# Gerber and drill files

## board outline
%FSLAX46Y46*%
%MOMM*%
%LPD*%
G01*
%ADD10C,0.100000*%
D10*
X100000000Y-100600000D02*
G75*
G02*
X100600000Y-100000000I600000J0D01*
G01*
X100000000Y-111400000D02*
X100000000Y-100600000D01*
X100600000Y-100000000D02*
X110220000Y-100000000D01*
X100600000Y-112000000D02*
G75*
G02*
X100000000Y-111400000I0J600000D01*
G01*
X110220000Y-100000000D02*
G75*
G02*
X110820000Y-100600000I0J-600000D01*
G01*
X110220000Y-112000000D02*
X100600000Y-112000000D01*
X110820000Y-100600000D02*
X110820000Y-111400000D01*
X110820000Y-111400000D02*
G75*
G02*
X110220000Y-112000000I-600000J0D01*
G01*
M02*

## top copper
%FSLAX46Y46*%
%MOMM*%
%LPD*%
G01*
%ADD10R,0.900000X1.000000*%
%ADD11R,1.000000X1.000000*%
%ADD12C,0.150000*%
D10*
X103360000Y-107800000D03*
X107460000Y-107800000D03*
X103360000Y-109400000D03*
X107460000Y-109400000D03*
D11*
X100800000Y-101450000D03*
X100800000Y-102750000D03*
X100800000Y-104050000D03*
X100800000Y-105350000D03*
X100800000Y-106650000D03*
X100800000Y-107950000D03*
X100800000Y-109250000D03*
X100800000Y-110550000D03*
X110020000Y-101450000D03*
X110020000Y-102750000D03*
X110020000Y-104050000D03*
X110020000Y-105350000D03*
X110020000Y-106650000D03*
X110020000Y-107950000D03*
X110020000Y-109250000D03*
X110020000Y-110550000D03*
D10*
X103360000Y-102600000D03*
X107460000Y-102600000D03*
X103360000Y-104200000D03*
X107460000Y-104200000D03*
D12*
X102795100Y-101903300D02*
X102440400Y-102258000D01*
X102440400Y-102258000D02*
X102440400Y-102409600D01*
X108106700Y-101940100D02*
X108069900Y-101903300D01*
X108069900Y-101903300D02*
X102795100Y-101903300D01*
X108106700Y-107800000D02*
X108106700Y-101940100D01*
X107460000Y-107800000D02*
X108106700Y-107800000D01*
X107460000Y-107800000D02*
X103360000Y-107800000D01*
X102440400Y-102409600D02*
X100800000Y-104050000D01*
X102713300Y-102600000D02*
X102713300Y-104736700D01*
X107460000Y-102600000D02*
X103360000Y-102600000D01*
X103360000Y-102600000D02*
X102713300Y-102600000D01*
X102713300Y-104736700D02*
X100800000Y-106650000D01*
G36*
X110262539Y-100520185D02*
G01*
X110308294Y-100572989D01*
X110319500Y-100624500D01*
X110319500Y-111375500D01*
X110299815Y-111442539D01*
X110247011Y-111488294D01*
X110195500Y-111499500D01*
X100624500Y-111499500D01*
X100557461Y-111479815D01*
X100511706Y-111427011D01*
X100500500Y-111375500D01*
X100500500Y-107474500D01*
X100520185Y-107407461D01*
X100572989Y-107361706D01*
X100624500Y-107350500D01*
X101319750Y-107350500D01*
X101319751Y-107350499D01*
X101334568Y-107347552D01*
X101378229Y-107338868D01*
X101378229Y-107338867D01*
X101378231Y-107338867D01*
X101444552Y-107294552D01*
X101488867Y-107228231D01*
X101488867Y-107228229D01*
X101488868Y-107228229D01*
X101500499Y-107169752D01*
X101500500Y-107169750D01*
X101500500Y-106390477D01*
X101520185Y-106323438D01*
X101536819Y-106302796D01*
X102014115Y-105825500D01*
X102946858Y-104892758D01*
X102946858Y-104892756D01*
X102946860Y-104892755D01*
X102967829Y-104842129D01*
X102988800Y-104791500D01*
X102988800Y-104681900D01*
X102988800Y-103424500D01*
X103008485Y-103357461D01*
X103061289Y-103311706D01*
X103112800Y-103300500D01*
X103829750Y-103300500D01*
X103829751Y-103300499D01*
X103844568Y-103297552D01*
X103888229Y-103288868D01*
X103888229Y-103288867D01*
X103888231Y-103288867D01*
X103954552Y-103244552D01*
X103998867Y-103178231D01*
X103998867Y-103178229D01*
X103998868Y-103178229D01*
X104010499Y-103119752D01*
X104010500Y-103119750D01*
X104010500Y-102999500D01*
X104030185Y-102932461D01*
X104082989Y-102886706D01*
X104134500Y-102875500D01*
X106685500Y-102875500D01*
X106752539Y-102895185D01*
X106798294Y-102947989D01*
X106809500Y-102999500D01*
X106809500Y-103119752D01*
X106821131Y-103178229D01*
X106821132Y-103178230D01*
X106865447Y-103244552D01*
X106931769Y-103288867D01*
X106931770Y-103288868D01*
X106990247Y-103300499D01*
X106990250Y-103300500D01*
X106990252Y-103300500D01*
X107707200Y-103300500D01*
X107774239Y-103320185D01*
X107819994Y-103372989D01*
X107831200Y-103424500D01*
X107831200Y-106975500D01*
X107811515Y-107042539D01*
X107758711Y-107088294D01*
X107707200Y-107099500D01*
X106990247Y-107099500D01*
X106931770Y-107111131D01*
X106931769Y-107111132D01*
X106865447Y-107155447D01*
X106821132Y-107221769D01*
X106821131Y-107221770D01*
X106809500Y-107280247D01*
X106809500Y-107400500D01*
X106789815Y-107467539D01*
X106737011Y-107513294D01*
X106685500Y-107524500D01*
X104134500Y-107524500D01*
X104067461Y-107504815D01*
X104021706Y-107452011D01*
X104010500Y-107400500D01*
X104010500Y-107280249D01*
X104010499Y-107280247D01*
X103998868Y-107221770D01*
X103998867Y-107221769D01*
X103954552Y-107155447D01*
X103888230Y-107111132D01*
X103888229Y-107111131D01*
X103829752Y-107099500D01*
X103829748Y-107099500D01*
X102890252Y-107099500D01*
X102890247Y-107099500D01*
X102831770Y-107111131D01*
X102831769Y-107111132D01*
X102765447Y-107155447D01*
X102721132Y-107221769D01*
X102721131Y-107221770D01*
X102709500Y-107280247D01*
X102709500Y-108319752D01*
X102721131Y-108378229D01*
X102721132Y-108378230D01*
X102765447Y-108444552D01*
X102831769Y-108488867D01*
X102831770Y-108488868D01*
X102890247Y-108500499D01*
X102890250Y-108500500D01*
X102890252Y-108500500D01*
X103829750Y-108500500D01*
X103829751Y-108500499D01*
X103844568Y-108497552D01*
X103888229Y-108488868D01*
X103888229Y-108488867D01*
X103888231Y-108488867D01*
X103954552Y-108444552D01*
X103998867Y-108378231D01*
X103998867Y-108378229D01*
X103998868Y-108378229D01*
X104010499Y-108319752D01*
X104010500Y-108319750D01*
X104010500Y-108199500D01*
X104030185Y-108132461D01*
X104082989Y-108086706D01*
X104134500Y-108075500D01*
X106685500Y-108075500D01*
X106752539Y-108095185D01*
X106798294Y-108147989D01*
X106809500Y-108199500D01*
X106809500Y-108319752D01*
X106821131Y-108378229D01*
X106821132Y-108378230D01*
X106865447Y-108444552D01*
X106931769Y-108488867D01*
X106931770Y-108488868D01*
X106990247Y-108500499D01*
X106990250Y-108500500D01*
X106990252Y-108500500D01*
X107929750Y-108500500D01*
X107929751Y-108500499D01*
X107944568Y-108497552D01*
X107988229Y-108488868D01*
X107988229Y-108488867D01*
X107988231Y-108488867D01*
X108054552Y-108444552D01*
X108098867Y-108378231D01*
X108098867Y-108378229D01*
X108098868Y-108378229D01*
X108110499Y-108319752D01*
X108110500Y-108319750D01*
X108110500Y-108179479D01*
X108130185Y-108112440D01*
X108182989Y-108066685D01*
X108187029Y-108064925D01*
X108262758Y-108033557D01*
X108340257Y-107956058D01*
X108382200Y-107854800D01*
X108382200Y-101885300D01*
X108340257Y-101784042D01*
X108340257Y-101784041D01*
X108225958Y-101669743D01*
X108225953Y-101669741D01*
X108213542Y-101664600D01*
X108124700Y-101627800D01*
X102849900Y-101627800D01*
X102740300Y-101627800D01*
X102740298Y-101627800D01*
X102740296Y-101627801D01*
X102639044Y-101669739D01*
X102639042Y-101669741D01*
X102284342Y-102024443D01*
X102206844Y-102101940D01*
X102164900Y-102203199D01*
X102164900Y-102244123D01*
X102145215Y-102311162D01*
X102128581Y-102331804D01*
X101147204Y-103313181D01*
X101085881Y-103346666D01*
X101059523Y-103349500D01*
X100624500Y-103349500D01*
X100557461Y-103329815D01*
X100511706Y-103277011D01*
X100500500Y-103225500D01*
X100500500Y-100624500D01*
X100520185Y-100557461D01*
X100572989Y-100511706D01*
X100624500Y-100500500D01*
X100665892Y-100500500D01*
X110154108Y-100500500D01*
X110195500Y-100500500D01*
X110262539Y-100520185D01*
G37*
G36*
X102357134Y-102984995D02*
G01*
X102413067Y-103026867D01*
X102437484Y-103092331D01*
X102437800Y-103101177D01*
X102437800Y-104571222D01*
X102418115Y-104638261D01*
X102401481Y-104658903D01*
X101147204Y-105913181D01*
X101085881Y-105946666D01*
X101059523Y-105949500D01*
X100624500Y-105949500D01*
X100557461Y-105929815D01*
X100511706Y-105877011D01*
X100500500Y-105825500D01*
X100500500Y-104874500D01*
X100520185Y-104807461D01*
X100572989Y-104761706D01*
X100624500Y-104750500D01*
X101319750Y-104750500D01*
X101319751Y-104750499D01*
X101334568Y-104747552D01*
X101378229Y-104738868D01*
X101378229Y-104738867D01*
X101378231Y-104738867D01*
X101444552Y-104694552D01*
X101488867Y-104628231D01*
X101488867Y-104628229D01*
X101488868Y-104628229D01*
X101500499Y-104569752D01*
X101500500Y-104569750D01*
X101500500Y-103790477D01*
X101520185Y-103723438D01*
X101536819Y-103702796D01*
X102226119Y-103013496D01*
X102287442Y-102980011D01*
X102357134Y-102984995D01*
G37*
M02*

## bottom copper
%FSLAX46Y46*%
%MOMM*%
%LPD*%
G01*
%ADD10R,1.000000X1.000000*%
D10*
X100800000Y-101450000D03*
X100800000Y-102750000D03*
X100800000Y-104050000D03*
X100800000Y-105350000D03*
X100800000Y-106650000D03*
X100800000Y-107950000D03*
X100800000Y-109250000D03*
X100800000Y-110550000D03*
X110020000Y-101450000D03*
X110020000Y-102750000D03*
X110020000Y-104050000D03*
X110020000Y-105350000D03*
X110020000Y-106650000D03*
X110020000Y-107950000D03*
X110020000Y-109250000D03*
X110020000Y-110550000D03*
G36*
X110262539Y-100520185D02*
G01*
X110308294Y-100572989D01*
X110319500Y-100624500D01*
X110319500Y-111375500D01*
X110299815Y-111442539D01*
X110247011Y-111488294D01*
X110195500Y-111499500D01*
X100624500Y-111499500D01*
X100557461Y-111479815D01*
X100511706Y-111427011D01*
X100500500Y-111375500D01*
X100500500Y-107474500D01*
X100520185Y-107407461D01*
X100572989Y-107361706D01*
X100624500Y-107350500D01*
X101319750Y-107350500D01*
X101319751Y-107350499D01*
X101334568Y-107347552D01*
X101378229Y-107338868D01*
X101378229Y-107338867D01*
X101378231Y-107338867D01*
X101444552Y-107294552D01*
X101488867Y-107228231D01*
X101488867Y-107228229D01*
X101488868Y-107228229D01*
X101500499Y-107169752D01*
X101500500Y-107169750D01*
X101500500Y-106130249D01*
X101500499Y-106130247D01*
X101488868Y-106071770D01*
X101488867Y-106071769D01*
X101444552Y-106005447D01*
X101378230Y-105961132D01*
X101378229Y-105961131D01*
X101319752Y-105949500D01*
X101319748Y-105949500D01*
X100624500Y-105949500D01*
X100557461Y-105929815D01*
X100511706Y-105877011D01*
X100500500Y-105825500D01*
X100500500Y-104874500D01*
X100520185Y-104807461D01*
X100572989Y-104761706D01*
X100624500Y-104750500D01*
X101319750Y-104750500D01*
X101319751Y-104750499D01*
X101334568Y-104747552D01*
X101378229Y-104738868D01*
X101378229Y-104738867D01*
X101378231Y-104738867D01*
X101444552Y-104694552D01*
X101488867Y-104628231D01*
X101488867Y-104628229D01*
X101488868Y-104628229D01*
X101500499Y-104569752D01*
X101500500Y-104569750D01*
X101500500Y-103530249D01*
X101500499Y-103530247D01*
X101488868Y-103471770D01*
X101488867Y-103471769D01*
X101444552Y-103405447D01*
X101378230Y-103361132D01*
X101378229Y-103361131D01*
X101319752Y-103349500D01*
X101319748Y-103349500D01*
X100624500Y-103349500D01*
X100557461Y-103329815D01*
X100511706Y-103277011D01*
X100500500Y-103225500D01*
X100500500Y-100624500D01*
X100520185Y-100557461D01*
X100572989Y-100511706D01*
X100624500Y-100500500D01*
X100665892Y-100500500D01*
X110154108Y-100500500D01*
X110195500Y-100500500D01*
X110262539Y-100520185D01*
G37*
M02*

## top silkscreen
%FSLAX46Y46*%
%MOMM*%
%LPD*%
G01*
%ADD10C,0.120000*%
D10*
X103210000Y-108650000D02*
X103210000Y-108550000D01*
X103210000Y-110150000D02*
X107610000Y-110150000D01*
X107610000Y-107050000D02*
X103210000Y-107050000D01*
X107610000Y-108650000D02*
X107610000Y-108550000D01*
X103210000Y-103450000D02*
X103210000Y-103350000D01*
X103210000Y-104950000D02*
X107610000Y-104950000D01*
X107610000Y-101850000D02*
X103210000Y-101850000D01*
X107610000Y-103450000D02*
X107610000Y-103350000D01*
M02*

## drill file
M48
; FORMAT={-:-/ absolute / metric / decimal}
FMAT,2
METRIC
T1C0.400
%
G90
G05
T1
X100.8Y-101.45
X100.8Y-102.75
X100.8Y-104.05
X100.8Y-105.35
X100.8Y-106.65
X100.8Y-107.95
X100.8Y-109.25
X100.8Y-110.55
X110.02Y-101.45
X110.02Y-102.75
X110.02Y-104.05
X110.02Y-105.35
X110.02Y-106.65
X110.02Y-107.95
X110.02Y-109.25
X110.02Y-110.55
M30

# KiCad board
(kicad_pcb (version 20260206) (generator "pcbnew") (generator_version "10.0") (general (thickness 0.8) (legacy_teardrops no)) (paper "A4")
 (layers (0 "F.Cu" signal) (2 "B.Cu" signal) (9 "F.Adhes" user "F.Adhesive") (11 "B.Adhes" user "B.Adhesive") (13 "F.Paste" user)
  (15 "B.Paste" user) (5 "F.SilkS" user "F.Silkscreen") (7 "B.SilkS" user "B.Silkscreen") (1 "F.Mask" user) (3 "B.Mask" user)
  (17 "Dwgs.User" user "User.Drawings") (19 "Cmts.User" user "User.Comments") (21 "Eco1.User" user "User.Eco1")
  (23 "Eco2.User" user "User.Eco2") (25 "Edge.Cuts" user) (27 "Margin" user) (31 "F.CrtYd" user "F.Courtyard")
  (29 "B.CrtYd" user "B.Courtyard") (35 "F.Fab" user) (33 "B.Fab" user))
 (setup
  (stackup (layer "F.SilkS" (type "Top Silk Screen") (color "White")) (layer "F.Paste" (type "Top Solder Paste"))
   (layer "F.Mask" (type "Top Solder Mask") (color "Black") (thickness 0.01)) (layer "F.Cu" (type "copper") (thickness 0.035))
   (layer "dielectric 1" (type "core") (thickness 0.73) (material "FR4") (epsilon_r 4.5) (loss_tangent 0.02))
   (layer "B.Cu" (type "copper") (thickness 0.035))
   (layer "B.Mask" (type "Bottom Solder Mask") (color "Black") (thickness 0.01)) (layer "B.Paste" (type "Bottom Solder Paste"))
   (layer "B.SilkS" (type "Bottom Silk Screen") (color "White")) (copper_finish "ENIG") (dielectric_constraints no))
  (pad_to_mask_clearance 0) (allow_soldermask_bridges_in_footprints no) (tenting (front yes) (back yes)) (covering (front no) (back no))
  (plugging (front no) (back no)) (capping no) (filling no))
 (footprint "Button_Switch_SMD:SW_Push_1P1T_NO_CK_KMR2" (layer "F.Cu") (at 105.41 108.6)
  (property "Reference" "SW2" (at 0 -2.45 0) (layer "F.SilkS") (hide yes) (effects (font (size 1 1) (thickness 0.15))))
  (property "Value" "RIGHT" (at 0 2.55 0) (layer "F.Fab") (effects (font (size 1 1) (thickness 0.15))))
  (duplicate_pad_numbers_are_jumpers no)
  (fp_line (start -2.2 0.05) (end -2.2 -0.05) (stroke (width 0.12) (type solid)) (layer "F.SilkS"))
  (fp_line (start -2.2 1.55) (end 2.2 1.55) (stroke (width 0.12) (type solid)) (layer "F.SilkS"))
  (fp_line (start 2.2 -1.55) (end -2.2 -1.55) (stroke (width 0.12) (type solid)) (layer "F.SilkS"))
  (fp_line (start 2.2 0.05) (end 2.2 -0.05) (stroke (width 0.12) (type solid)) (layer "F.SilkS"))
  (pad "1" smd rect (at -2.05 -0.8) (size 0.9 1) (layers "F.Cu" "F.Mask" "F.Paste") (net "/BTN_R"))
  (pad "1" smd rect (at 2.05 -0.8) (size 0.9 1) (layers "F.Cu" "F.Mask" "F.Paste") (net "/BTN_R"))
  (pad "2" smd rect (at -2.05 0.8) (size 0.9 1) (layers "F.Cu" "F.Mask" "F.Paste") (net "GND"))
  (pad "2" smd rect (at 2.05 0.8) (size 0.9 1) (layers "F.Cu" "F.Mask" "F.Paste") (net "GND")))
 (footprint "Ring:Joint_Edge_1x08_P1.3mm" (layer "F.Cu") (at 100.8 106)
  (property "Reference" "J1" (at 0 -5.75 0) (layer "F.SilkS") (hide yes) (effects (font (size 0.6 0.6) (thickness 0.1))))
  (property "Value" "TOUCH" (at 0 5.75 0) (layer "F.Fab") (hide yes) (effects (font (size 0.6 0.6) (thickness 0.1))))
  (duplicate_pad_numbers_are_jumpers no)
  (pad "1" thru_hole rect (at 0 -4.55) (size 1 1) (drill 0.4) (layers "*.Cu" "*.Mask") (remove_unused_layers no) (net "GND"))
  (pad "2" thru_hole rect (at 0 -3.25) (size 1 1) (drill 0.4) (layers "*.Cu" "*.Mask") (remove_unused_layers no) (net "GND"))
  (pad "3" thru_hole rect (at 0 -1.95) (size 1 1) (drill 0.4) (layers "*.Cu" "*.Mask") (remove_unused_layers no) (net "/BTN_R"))
  (pad "4" thru_hole rect (at 0 -0.65) (size 1 1) (drill 0.4) (layers "*.Cu" "*.Mask") (remove_unused_layers no) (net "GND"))
  (pad "5" thru_hole rect (at 0 0.65) (size 1 1) (drill 0.4) (layers "*.Cu" "*.Mask") (remove_unused_layers no) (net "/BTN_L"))
  (pad "6" thru_hole rect (at 0 1.95) (size 1 1) (drill 0.4) (layers "*.Cu" "*.Mask") (remove_unused_layers no) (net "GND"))
  (pad "7" thru_hole rect (at 0 3.25) (size 1 1) (drill 0.4) (layers "*.Cu" "*.Mask") (remove_unused_layers no) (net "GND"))
  (pad "8" thru_hole rect (at 0 4.55) (size 1 1) (drill 0.4) (layers "*.Cu" "*.Mask") (remove_unused_layers no) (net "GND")))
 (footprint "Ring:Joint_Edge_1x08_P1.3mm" (layer "F.Cu") (at 110.02 106)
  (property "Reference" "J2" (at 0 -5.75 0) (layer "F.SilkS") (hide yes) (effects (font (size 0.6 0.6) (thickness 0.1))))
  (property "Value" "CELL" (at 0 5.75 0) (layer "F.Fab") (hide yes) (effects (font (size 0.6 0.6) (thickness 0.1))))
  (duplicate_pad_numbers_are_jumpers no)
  (pad "1" thru_hole rect (at 0 -4.55) (size 1 1) (drill 0.4) (layers "*.Cu" "*.Mask") (remove_unused_layers no) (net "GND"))
  (pad "2" thru_hole rect (at 0 -3.25) (size 1 1) (drill 0.4) (layers "*.Cu" "*.Mask") (remove_unused_layers no) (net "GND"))
  (pad "3" thru_hole rect (at 0 -1.95) (size 1 1) (drill 0.4) (layers "*.Cu" "*.Mask") (remove_unused_layers no) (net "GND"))
  (pad "4" thru_hole rect (at 0 -0.65) (size 1 1) (drill 0.4) (layers "*.Cu" "*.Mask") (remove_unused_layers no) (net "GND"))
  (pad "5" thru_hole rect (at 0 0.65) (size 1 1) (drill 0.4) (layers "*.Cu" "*.Mask") (remove_unused_layers no) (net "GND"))
  (pad "6" thru_hole rect (at 0 1.95) (size 1 1) (drill 0.4) (layers "*.Cu" "*.Mask") (remove_unused_layers no) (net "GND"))
  (pad "7" thru_hole rect (at 0 3.25) (size 1 1) (drill 0.4) (layers "*.Cu" "*.Mask") (remove_unused_layers no) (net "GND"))
  (pad "8" thru_hole rect (at 0 4.55) (size 1 1) (drill 0.4) (layers "*.Cu" "*.Mask") (remove_unused_layers no) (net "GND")))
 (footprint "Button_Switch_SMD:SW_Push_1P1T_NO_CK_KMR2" (layer "F.Cu") (at 105.41 103.4)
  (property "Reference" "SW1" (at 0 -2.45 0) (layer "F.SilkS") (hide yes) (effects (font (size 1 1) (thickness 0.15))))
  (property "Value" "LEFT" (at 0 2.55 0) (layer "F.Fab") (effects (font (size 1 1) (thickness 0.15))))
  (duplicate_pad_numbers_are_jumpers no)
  (fp_line (start -2.2 0.05) (end -2.2 -0.05) (stroke (width 0.12) (type solid)) (layer "F.SilkS"))
  (fp_line (start -2.2 1.55) (end 2.2 1.55) (stroke (width 0.12) (type solid)) (layer "F.SilkS"))
  (fp_line (start 2.2 -1.55) (end -2.2 -1.55) (stroke (width 0.12) (type solid)) (layer "F.SilkS"))
  (fp_line (start 2.2 0.05) (end 2.2 -0.05) (stroke (width 0.12) (type solid)) (layer "F.SilkS"))
  (pad "1" smd rect (at -2.05 -0.8) (size 0.9 1) (layers "F.Cu" "F.Mask" "F.Paste") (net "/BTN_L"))
  (pad "1" smd rect (at 2.05 -0.8) (size 0.9 1) (layers "F.Cu" "F.Mask" "F.Paste") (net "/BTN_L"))
  (pad "2" smd rect (at -2.05 0.8) (size 0.9 1) (layers "F.Cu" "F.Mask" "F.Paste") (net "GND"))
  (pad "2" smd rect (at 2.05 0.8) (size 0.9 1) (layers "F.Cu" "F.Mask" "F.Paste") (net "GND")))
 (gr_arc (start 100 100.6) (mid 100.175736 100.175736) (end 100.6 100) (stroke (width 0.1) (type default)) (layer "Edge.Cuts"))
 (gr_line (start 100 111.4) (end 100 100.6) (stroke (width 0.1) (type default)) (layer "Edge.Cuts"))
 (gr_line (start 100.6 100) (end 110.22 100) (stroke (width 0.1) (type default)) (layer "Edge.Cuts"))
 (gr_arc (start 100.6 112) (mid 100.175736 111.824264) (end 100 111.4) (stroke (width 0.1) (type default)) (layer "Edge.Cuts"))
 (gr_arc (start 110.22 100) (mid 110.644264 100.175736) (end 110.82 100.6) (stroke (width 0.1) (type default)) (layer "Edge.Cuts"))
 (gr_line (start 110.22 112) (end 100.6 112) (stroke (width 0.1) (type default)) (layer "Edge.Cuts"))
 (gr_line (start 110.82 100.6) (end 110.82 111.4) (stroke (width 0.1) (type default)) (layer "Edge.Cuts"))
 (gr_arc (start 110.82 111.4) (mid 110.644264 111.824264) (end 110.22 112) (stroke (width 0.1) (type default)) (layer "Edge.Cuts"))
 (segment (start 102.7951 101.9033) (end 102.4404 102.258) (width 0.15) (layer "F.Cu") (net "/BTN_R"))
 (segment (start 102.4404 102.258) (end 102.4404 102.4096) (width 0.15) (layer "F.Cu") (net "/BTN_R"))
 (segment (start 108.1067 101.9401) (end 108.0699 101.9033) (width 0.15) (layer "F.Cu") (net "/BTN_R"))
 (segment (start 108.0699 101.9033) (end 102.7951 101.9033) (width 0.15) (layer "F.Cu") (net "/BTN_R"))
 (segment (start 108.1067 107.8) (end 108.1067 101.9401) (width 0.15) (layer "F.Cu") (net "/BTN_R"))
 (segment (start 107.46 107.8) (end 108.1067 107.8) (width 0.15) (layer "F.Cu") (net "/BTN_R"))
 (segment (start 107.46 107.8) (end 103.36 107.8) (width 0.15) (layer "F.Cu") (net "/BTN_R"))
 (segment (start 102.4404 102.4096) (end 100.8 104.05) (width 0.15) (layer "F.Cu") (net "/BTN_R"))
 (segment (start 102.7133 102.6) (end 102.7133 104.7367) (width 0.15) (layer "F.Cu") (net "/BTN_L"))
 (segment (start 107.46 102.6) (end 103.36 102.6) (width 0.15) (layer "F.Cu") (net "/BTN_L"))
 (segment (start 103.36 102.6) (end 102.7133 102.6) (width 0.15) (layer "F.Cu") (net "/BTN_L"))
 (segment (start 102.7133 104.7367) (end 100.8 106.65) (width 0.15) (layer "F.Cu") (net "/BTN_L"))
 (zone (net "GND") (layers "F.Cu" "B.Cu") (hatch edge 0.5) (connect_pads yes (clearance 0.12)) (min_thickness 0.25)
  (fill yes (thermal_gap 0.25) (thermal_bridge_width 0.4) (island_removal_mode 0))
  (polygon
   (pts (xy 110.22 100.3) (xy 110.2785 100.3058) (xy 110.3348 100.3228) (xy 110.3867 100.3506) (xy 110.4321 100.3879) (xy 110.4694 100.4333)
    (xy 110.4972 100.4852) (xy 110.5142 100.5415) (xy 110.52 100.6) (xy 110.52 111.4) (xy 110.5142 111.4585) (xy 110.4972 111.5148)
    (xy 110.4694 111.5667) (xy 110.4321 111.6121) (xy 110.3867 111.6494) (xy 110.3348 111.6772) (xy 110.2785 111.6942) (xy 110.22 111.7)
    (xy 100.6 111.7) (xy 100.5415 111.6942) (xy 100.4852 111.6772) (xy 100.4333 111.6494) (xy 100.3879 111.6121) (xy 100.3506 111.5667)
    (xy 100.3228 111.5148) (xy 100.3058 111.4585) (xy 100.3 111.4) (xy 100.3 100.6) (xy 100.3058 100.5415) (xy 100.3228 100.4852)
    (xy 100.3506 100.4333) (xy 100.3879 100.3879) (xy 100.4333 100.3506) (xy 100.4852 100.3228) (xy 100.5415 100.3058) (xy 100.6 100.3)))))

